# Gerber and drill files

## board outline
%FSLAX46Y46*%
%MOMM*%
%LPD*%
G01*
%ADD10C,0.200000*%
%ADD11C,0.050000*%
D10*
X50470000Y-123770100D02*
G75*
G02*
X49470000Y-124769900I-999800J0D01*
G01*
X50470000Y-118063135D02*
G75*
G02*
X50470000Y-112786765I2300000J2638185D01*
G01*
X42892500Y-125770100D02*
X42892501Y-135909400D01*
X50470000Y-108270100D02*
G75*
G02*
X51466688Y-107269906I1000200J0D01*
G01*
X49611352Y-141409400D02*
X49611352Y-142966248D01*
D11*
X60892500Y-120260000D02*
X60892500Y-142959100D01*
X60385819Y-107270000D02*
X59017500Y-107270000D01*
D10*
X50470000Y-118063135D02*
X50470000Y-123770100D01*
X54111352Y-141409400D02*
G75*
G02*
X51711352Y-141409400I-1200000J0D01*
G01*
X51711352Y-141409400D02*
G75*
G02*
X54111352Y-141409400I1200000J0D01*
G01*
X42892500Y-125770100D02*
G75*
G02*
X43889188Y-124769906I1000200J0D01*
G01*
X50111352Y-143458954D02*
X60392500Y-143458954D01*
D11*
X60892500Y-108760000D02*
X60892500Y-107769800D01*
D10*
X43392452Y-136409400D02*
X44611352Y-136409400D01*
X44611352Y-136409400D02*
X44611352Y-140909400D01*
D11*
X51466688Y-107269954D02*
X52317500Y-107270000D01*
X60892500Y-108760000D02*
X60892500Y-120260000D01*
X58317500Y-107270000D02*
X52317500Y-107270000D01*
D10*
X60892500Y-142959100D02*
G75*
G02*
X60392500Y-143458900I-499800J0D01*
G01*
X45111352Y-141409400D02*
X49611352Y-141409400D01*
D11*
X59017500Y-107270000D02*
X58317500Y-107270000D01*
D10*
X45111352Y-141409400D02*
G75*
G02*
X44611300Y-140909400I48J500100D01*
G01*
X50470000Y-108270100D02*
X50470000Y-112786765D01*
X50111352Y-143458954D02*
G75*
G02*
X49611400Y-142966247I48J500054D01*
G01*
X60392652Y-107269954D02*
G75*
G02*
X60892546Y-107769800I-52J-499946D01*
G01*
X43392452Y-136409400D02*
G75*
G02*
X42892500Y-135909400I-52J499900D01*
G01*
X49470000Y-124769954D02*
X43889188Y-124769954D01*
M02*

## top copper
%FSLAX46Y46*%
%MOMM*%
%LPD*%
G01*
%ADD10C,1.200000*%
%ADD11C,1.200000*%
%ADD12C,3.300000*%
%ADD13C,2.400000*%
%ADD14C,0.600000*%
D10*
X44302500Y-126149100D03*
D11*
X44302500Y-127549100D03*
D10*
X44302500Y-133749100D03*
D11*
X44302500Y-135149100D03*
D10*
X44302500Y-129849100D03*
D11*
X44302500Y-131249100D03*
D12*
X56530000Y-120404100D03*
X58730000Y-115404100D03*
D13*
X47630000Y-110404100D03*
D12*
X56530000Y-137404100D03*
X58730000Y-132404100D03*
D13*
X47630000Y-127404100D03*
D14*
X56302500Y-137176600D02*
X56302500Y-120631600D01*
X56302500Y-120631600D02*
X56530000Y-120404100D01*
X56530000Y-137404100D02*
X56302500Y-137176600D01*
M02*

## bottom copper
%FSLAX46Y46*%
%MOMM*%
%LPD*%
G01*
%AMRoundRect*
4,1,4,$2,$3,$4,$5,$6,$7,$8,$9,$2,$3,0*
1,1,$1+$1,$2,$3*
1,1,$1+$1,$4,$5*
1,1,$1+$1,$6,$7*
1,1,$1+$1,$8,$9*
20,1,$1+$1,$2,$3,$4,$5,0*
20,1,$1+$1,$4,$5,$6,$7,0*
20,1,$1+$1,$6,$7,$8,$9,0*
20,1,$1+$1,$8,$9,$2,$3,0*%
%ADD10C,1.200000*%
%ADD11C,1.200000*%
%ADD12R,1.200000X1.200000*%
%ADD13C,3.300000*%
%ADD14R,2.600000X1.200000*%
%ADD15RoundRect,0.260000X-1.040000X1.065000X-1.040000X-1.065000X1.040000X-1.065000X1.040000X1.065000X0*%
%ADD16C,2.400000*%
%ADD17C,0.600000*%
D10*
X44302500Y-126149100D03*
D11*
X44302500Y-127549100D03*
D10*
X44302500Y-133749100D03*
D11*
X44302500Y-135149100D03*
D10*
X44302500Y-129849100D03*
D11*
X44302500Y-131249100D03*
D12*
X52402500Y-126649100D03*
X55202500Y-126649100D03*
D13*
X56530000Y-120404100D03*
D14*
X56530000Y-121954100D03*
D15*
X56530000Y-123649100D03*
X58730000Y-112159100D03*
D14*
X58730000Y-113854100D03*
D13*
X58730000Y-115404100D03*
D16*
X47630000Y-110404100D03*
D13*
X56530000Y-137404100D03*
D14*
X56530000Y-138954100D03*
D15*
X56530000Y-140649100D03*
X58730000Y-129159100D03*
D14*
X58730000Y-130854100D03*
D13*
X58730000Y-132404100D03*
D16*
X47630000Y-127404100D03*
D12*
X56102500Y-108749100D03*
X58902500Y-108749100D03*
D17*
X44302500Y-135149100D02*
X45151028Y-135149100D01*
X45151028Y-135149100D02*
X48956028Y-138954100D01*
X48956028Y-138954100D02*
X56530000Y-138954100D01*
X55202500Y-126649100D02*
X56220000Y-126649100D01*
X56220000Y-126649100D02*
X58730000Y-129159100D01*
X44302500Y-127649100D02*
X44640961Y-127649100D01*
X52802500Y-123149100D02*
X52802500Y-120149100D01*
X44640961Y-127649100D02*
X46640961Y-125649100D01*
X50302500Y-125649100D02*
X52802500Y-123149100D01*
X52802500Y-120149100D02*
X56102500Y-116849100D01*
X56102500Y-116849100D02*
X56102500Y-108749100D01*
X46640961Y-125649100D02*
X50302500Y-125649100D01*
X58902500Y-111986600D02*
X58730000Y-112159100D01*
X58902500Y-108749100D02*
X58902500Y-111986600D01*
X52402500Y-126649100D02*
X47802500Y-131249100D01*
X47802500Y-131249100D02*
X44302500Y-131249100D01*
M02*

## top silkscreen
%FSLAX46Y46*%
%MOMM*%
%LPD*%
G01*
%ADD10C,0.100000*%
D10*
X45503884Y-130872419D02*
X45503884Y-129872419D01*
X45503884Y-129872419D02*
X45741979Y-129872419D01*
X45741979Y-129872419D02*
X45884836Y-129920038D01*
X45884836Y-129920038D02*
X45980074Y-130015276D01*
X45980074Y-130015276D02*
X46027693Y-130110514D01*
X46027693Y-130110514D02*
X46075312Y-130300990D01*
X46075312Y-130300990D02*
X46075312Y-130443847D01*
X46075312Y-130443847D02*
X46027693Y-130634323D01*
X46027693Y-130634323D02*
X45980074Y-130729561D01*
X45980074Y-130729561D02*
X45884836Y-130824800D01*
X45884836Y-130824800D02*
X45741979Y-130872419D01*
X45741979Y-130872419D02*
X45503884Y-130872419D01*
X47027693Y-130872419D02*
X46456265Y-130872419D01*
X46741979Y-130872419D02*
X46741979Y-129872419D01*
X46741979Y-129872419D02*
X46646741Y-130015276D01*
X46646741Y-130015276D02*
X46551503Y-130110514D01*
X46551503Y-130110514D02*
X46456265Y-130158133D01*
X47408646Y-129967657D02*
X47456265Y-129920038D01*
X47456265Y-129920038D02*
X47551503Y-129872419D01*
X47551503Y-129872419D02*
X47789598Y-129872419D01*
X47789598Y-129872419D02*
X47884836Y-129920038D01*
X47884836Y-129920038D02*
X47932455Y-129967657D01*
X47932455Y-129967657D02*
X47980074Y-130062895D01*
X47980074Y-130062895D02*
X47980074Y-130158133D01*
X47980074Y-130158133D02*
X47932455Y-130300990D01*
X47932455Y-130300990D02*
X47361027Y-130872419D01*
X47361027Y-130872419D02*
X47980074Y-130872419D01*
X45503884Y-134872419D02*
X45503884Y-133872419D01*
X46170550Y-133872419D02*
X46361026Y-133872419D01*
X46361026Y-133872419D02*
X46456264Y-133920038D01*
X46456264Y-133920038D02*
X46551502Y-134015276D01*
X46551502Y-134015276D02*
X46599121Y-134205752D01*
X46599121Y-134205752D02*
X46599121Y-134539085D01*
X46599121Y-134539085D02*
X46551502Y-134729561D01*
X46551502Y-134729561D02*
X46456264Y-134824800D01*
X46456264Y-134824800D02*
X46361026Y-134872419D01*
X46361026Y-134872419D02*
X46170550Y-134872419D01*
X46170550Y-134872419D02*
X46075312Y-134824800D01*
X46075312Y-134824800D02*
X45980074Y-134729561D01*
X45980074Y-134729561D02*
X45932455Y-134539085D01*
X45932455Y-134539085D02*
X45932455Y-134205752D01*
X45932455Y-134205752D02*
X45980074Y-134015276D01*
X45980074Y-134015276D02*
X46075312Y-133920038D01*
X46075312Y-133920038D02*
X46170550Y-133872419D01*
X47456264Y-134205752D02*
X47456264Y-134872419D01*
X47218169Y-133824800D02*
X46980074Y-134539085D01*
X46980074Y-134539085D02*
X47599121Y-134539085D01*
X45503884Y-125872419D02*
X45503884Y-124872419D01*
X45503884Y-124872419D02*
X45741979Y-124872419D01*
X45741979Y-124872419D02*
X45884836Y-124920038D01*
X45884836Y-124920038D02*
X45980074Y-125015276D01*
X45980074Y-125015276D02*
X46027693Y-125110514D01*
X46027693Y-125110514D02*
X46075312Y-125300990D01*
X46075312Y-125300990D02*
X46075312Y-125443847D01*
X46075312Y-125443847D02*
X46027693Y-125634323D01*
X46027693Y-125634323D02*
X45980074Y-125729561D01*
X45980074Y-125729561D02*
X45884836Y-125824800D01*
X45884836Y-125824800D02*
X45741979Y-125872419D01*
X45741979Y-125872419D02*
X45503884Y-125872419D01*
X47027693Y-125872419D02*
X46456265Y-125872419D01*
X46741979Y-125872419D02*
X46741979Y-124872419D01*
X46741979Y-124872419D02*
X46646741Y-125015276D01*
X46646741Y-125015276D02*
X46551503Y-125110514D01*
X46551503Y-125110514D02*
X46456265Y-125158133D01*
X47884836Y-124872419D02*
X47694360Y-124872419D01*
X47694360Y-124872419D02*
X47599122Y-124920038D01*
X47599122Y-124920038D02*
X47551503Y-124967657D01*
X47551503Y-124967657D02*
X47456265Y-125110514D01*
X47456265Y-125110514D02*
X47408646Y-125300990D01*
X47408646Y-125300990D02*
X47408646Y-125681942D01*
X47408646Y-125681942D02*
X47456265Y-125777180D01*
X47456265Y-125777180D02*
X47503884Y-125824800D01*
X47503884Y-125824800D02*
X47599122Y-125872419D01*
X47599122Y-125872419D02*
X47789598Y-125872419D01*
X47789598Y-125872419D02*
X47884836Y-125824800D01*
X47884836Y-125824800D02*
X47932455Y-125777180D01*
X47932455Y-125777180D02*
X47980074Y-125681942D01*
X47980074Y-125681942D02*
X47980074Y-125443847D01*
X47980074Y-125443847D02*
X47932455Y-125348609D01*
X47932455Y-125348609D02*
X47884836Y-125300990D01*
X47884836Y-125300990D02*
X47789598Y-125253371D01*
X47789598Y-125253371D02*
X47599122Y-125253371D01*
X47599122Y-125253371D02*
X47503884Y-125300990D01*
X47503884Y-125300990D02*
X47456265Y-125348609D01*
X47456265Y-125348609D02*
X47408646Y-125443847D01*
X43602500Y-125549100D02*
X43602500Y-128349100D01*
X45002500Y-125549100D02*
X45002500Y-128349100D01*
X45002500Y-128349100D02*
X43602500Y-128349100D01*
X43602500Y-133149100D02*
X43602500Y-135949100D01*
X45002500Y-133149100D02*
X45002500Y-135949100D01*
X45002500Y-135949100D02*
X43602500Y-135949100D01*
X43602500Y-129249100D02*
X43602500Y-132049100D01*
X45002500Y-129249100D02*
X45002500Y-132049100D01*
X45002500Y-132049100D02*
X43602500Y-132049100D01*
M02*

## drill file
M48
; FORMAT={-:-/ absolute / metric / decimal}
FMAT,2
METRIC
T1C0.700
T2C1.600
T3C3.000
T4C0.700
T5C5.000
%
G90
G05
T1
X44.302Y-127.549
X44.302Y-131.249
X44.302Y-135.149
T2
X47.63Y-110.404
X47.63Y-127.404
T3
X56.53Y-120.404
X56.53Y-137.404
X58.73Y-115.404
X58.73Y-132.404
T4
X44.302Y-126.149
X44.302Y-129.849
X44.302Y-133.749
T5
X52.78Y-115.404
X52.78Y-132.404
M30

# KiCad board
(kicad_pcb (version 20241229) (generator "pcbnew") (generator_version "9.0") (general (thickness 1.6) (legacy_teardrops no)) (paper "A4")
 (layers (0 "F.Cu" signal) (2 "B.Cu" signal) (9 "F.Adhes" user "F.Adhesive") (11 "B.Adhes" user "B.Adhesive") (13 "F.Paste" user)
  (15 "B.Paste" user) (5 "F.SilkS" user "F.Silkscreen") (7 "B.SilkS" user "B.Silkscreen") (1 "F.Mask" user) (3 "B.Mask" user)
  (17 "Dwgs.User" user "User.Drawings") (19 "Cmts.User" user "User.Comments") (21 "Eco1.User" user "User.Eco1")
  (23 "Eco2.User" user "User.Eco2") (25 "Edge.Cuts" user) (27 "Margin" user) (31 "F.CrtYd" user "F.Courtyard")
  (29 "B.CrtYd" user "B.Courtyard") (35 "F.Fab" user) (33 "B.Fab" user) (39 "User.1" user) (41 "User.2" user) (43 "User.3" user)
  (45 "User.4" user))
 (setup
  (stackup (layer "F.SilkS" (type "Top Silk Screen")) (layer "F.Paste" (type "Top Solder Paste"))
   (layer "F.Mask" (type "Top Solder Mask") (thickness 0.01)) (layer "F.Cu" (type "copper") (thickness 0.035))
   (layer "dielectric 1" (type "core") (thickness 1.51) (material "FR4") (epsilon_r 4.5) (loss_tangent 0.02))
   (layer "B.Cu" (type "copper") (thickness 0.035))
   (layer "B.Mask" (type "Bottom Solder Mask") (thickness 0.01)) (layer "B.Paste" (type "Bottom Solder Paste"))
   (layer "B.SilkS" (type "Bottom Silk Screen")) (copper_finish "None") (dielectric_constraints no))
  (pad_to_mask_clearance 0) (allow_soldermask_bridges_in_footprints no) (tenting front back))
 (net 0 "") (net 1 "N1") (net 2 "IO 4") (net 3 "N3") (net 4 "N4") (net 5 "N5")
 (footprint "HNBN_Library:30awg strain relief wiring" (layer "F.Cu") (at 44.3025 127.5491 -90)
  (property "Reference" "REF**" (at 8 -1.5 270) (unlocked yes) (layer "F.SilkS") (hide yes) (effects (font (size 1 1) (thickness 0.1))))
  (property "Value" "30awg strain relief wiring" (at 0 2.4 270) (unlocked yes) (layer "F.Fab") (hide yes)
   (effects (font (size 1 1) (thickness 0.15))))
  (fp_line (start -2 0.7) (end 0.8 0.7) (stroke (width 0.1) (type default)) (layer "F.SilkS"))
  (fp_line (start -2 -0.7) (end 0.8 -0.7) (stroke (width 0.1) (type default)) (layer "F.SilkS"))
  (fp_line (start 0.8 -0.7) (end 0.8 0.7) (stroke (width 0.1) (type default)) (layer "F.SilkS"))
  (pad "" np_thru_hole circle (at -1.4 0 270) (size 1.2 1.2) (drill 0.7) (layers "*.Cu" "*.Mask")
   (teardrops (best_length_ratio 0.5) (max_length 1) (best_width_ratio 0.6) (max_width 2) (curved_edges no) (filter_ratio 0.9) (enabled no)
    (allow_two_segments yes) (prefer_zone_connections yes)))
  (pad "1" thru_hole circle (at 0 0 270) (size 1.2 1.2) (drill 0.7) (layers "*.Cu" "*.Mask") (remove_unused_layers no) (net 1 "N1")))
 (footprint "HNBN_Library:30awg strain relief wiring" (layer "F.Cu") (at 44.3025 135.1491 -90)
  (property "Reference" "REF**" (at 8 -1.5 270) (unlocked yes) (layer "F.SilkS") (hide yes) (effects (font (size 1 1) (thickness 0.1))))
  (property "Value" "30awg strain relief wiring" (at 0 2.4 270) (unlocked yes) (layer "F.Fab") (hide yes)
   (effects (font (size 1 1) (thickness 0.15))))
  (fp_line (start -2 0.7) (end 0.8 0.7) (stroke (width 0.1) (type default)) (layer "F.SilkS"))
  (fp_line (start -2 -0.7) (end 0.8 -0.7) (stroke (width 0.1) (type default)) (layer "F.SilkS"))
  (fp_line (start 0.8 -0.7) (end 0.8 0.7) (stroke (width 0.1) (type default)) (layer "F.SilkS"))
  (pad "" np_thru_hole circle (at -1.4 0 270) (size 1.2 1.2) (drill 0.7) (layers "*.Cu" "*.Mask")
   (teardrops (best_length_ratio 0.5) (max_length 1) (best_width_ratio 0.6) (max_width 2) (curved_edges no) (filter_ratio 0.9) (enabled no)
    (allow_two_segments yes) (prefer_zone_connections yes)))
  (pad "1" thru_hole circle (at 0 0 270) (size 1.2 1.2) (drill 0.7) (layers "*.Cu" "*.Mask") (remove_unused_layers no) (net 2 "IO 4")))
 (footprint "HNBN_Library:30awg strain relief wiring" (layer "F.Cu") (at 44.3025 131.2491 -90)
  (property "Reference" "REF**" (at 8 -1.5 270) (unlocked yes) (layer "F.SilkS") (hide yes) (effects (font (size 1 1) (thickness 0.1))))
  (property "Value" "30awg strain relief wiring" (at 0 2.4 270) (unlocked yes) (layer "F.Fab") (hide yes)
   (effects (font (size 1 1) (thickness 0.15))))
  (fp_line (start -2 0.7) (end 0.8 0.7) (stroke (width 0.1) (type default)) (layer "F.SilkS"))
  (fp_line (start -2 -0.7) (end 0.8 -0.7) (stroke (width 0.1) (type default)) (layer "F.SilkS"))
  (fp_line (start 0.8 -0.7) (end 0.8 0.7) (stroke (width 0.1) (type default)) (layer "F.SilkS"))
  (pad "" np_thru_hole circle (at -1.4 0 270) (size 1.2 1.2) (drill 0.7) (layers "*.Cu" "*.Mask")
   (teardrops (best_length_ratio 0.5) (max_length 1) (best_width_ratio 0.6) (max_width 2) (curved_edges no) (filter_ratio 0.9) (enabled no)
    (allow_two_segments yes) (prefer_zone_connections yes)))
  (pad "1" thru_hole circle (at 0 0 270) (size 1.2 1.2) (drill 0.7) (layers "*.Cu" "*.Mask") (remove_unused_layers no) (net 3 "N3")))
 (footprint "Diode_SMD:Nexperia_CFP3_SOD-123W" (layer "B.Cu") (at 53.8025 126.6491)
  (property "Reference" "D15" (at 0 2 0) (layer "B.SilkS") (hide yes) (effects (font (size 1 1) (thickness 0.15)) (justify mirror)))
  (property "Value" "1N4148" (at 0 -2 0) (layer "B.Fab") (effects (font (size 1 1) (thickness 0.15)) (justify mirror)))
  (pad "1" smd rect (at -1.4 0) (size 1.2 1.2) (layers "B.Cu" "B.Mask" "B.Paste") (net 3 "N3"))
  (pad "2" smd rect (at 1.4 0) (size 1.2 1.2) (layers "B.Cu" "B.Mask" "B.Paste") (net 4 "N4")))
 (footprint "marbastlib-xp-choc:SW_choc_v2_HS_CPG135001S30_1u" (layer "B.Cu") (at 52.78 115.4041 -90)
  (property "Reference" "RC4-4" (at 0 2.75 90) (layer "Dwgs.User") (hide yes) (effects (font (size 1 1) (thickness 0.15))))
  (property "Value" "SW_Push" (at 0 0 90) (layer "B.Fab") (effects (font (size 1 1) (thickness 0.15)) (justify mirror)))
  (pad "" np_thru_hole circle (at 0 0 90) (size 5 5) (drill 5) (layers "*.Cu" "*.Mask"))
  (pad "1" thru_hole circle (at 5 -3.75 270) (size 3.3 3.3) (drill 3) (layers "*.Cu" "B.Mask") (remove_unused_layers no) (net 2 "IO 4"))
  (pad "1" smd rect (at 6.55 -3.75 270) (size 1.2 2.6) (layers "B.Cu") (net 2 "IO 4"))
  (pad "1" smd roundrect (at 8.245 -3.75 270) (size 2.65 2.6) (layers "B.Cu" "B.Mask" "B.Paste") (roundrect_rratio 0.1) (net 2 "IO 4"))
  (pad "2" smd roundrect (at -3.245 -5.95 270) (size 2.65 2.6) (layers "B.Cu" "B.Mask" "B.Paste") (roundrect_rratio 0.1) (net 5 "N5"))
  (pad "2" smd rect (at -1.55 -5.95 90) (size 1.2 2.6) (layers "B.Cu") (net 5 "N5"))
  (pad "2" thru_hole circle (at 0 -5.95 270) (size 3.3 3.3) (drill 3) (layers "*.Cu" "B.Mask") (remove_unused_layers no) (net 5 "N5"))
  (pad "MP" thru_hole circle (at -5 5.15 90) (size 2.4 2.4) (drill 1.6) (layers "*.Cu" "B.Mask") (remove_unused_layers no)))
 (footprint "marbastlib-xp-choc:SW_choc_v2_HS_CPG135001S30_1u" (layer "B.Cu") (at 52.78 132.4041 -90)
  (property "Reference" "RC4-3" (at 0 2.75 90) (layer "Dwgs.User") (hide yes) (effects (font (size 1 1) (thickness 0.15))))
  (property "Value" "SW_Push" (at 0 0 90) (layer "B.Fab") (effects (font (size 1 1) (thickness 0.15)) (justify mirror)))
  (pad "" np_thru_hole circle (at 0 0 90) (size 5 5) (drill 5) (layers "*.Cu" "*.Mask"))
  (pad "1" thru_hole circle (at 5 -3.75 270) (size 3.3 3.3) (drill 3) (layers "*.Cu" "B.Mask") (remove_unused_layers no) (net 2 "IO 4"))
  (pad "1" smd rect (at 6.55 -3.75 270) (size 1.2 2.6) (layers "B.Cu") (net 2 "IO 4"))
  (pad "1" smd roundrect (at 8.245 -3.75 270) (size 2.65 2.6) (layers "B.Cu" "B.Mask" "B.Paste") (roundrect_rratio 0.1) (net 2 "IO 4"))
  (pad "2" smd roundrect (at -3.245 -5.95 270) (size 2.65 2.6) (layers "B.Cu" "B.Mask" "B.Paste") (roundrect_rratio 0.1) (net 4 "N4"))
  (pad "2" smd rect (at -1.55 -5.95 90) (size 1.2 2.6) (layers "B.Cu") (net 4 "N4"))
  (pad "2" thru_hole circle (at 0 -5.95 270) (size 3.3 3.3) (drill 3) (layers "*.Cu" "B.Mask") (remove_unused_layers no) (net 4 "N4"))
  (pad "MP" thru_hole circle (at -5 5.15 90) (size 2.4 2.4) (drill 1.6) (layers "*.Cu" "B.Mask") (remove_unused_layers no)))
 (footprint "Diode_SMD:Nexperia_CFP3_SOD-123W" (layer "B.Cu") (at 57.5025 108.7491)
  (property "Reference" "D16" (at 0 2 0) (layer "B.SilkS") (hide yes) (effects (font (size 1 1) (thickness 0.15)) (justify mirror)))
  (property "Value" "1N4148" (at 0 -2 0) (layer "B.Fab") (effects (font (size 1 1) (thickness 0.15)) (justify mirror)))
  (pad "1" smd rect (at -1.4 0) (size 1.2 1.2) (layers "B.Cu" "B.Mask" "B.Paste") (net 1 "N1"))
  (pad "2" smd rect (at 1.4 0) (size 1.2 1.2) (layers "B.Cu" "B.Mask" "B.Paste") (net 5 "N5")))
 (gr_arc (start 50.47 123.7701) (mid 50.177101 124.477171) (end 49.47 124.769954) (stroke (width 0.2) (type default)) (layer "Edge.Cuts"))
 (gr_arc (start 50.47 118.063135) (mid 49.269997 115.42495) (end 50.47 112.786765) (stroke (width 0.2) (type default)) (layer "Edge.Cuts"))
 (gr_line (start 42.8925 125.7701) (end 42.892501 135.9094) (stroke (width 0.2) (type default)) (layer "Edge.Cuts"))
 (gr_arc (start 50.47 108.2701) (mid 50.761717 107.56413) (end 51.466688 107.269954) (stroke (width 0.2) (type default)) (layer "Edge.Cuts"))
 (gr_line (start 49.611352 141.4094) (end 49.611352 142.966248) (stroke (width 0.2) (type default)) (layer "Edge.Cuts"))
 (gr_line (start 60.8925 120.26) (end 60.8925 142.9591) (stroke (width 0.05) (type default)) (layer "Edge.Cuts"))
 (gr_line (start 60.385819 107.27) (end 59.0175 107.27) (stroke (width 0.05) (type default)) (layer "Edge.Cuts"))
 (gr_line (start 50.47 118.063135) (end 50.47 123.7701) (stroke (width 0.2) (type default)) (layer "Edge.Cuts"))
 (gr_circle (center 52.911352 141.4094) (end 54.111352 141.4094) (stroke (width 0.2) (type default)) (fill no) (layer "Edge.Cuts"))
 (gr_arc (start 42.8925 125.7701) (mid 43.184217 125.06413) (end 43.889188 124.769954) (stroke (width 0.2) (type default))
  (layer "Edge.Cuts"))
 (gr_line (start 50.111352 143.458954) (end 60.3925 143.458954) (stroke (width 0.2) (type default)) (layer "Edge.Cuts"))
 (gr_line (start 60.8925 108.76) (end 60.8925 107.7698) (stroke (width 0.05) (type default)) (layer "Edge.Cuts"))
 (gr_line (start 43.392452 136.4094) (end 44.611352 136.4094) (stroke (width 0.2) (type default)) (layer "Edge.Cuts"))
 (gr_line (start 44.611352 136.4094) (end 44.611352 140.9094) (stroke (width 0.2) (type default)) (layer "Edge.Cuts"))
 (gr_line (start 51.466688 107.269954) (end 52.3175 107.27) (stroke (width 0.05) (type default)) (layer "Edge.Cuts"))
 (gr_line (start 60.8925 108.76) (end 60.8925 120.26) (stroke (width 0.05) (type default)) (layer "Edge.Cuts"))
 (gr_line (start 58.3175 107.27) (end 52.3175 107.27) (stroke (width 0.05) (type default)) (layer "Edge.Cuts"))
 (gr_arc (start 60.8925 142.9591) (mid 60.746047 143.312618) (end 60.3925 143.458954) (stroke (width 0.2) (type default))
  (layer "Edge.Cuts"))
 (gr_line (start 45.111352 141.4094) (end 49.611352 141.4094) (stroke (width 0.2) (type default)) (layer "Edge.Cuts"))
 (gr_line (start 59.0175 107.27) (end 58.3175 107.27) (stroke (width 0.05) (type default)) (layer "Edge.Cuts"))
 (gr_arc (start 45.111352 141.4094) (mid 44.75783 141.262936) (end 44.611352 140.9094) (stroke (width 0.2) (type default))
  (layer "Edge.Cuts"))
 (gr_line (start 50.47 108.2701) (end 50.47 112.786765) (stroke (width 0.2) (type default)) (layer "Edge.Cuts"))
 (gr_arc (start 50.111352 143.458954) (mid 49.760364 143.315069) (end 49.611352 142.966248) (stroke (width 0.2) (type default))
  (layer "Edge.Cuts"))
 (gr_arc (start 60.392652 107.269954) (mid 60.746063 107.416374) (end 60.8925 107.7698) (stroke (width 0.2) (type default))
  (layer "Edge.Cuts"))
 (gr_arc (start 43.392452 136.4094) (mid 43.0389 136.262966) (end 42.8925 135.9094) (stroke (width 0.2) (type default)) (layer "Edge.Cuts"))
 (gr_line (start 49.47 124.769954) (end 43.889188 124.769954) (stroke (width 0.2) (type default)) (layer "Edge.Cuts"))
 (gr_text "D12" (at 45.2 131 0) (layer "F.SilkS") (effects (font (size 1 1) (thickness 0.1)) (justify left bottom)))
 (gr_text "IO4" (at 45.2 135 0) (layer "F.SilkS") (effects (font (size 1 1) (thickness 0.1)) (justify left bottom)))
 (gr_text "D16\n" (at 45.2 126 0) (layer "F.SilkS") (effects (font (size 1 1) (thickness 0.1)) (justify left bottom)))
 (segment (start 56.3025 137.1766) (end 56.3025 120.6316) (width 0.6) (layer "F.Cu") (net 2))
 (segment (start 56.3025 120.6316) (end 56.53 120.4041) (width 0.6) (layer "F.Cu") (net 2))
 (segment (start 56.53 137.4041) (end 56.3025 137.1766) (width 0.6) (layer "F.Cu") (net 2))
 (segment (start 44.3025 135.1491) (end 45.151028 135.1491) (width 0.6) (layer "B.Cu") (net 2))
 (segment (start 45.151028 135.1491) (end 48.956028 138.9541) (width 0.6) (layer "B.Cu") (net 2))
 (segment (start 48.956028 138.9541) (end 56.53 138.9541) (width 0.6) (layer "B.Cu") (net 2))
 (segment (start 55.2025 126.6491) (end 56.22 126.6491) (width 0.6) (layer "B.Cu") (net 4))
 (segment (start 56.22 126.6491) (end 58.73 129.1591) (width 0.6) (layer "B.Cu") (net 4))
 (segment (start 44.3025 127.6491) (end 44.640961 127.6491) (width 0.6) (layer "B.Cu") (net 1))
 (segment (start 52.8025 123.1491) (end 52.8025 120.1491) (width 0.6) (layer "B.Cu") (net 1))
 (segment (start 44.640961 127.6491) (end 46.640961 125.6491) (width 0.6) (layer "B.Cu") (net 1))
 (segment (start 50.3025 125.6491) (end 52.8025 123.1491) (width 0.6) (layer "B.Cu") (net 1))
 (segment (start 52.8025 120.1491) (end 56.1025 116.8491) (width 0.6) (layer "B.Cu") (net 1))
 (segment (start 56.1025 116.8491) (end 56.1025 108.7491) (width 0.6) (layer "B.Cu") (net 1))
 (segment (start 46.640961 125.6491) (end 50.3025 125.6491) (width 0.6) (layer "B.Cu") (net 1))
 (segment (start 58.9025 111.9866) (end 58.73 112.1591) (width 0.6) (layer "B.Cu") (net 5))
 (segment (start 58.9025 108.7491) (end 58.9025 111.9866) (width 0.6) (layer "B.Cu") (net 5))
 (segment (start 52.4025 126.6491) (end 47.8025 131.2491) (width 0.6) (layer "B.Cu") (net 3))
 (segment (start 47.8025 131.2491) (end 44.3025 131.2491) (width 0.6) (layer "B.Cu") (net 3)))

